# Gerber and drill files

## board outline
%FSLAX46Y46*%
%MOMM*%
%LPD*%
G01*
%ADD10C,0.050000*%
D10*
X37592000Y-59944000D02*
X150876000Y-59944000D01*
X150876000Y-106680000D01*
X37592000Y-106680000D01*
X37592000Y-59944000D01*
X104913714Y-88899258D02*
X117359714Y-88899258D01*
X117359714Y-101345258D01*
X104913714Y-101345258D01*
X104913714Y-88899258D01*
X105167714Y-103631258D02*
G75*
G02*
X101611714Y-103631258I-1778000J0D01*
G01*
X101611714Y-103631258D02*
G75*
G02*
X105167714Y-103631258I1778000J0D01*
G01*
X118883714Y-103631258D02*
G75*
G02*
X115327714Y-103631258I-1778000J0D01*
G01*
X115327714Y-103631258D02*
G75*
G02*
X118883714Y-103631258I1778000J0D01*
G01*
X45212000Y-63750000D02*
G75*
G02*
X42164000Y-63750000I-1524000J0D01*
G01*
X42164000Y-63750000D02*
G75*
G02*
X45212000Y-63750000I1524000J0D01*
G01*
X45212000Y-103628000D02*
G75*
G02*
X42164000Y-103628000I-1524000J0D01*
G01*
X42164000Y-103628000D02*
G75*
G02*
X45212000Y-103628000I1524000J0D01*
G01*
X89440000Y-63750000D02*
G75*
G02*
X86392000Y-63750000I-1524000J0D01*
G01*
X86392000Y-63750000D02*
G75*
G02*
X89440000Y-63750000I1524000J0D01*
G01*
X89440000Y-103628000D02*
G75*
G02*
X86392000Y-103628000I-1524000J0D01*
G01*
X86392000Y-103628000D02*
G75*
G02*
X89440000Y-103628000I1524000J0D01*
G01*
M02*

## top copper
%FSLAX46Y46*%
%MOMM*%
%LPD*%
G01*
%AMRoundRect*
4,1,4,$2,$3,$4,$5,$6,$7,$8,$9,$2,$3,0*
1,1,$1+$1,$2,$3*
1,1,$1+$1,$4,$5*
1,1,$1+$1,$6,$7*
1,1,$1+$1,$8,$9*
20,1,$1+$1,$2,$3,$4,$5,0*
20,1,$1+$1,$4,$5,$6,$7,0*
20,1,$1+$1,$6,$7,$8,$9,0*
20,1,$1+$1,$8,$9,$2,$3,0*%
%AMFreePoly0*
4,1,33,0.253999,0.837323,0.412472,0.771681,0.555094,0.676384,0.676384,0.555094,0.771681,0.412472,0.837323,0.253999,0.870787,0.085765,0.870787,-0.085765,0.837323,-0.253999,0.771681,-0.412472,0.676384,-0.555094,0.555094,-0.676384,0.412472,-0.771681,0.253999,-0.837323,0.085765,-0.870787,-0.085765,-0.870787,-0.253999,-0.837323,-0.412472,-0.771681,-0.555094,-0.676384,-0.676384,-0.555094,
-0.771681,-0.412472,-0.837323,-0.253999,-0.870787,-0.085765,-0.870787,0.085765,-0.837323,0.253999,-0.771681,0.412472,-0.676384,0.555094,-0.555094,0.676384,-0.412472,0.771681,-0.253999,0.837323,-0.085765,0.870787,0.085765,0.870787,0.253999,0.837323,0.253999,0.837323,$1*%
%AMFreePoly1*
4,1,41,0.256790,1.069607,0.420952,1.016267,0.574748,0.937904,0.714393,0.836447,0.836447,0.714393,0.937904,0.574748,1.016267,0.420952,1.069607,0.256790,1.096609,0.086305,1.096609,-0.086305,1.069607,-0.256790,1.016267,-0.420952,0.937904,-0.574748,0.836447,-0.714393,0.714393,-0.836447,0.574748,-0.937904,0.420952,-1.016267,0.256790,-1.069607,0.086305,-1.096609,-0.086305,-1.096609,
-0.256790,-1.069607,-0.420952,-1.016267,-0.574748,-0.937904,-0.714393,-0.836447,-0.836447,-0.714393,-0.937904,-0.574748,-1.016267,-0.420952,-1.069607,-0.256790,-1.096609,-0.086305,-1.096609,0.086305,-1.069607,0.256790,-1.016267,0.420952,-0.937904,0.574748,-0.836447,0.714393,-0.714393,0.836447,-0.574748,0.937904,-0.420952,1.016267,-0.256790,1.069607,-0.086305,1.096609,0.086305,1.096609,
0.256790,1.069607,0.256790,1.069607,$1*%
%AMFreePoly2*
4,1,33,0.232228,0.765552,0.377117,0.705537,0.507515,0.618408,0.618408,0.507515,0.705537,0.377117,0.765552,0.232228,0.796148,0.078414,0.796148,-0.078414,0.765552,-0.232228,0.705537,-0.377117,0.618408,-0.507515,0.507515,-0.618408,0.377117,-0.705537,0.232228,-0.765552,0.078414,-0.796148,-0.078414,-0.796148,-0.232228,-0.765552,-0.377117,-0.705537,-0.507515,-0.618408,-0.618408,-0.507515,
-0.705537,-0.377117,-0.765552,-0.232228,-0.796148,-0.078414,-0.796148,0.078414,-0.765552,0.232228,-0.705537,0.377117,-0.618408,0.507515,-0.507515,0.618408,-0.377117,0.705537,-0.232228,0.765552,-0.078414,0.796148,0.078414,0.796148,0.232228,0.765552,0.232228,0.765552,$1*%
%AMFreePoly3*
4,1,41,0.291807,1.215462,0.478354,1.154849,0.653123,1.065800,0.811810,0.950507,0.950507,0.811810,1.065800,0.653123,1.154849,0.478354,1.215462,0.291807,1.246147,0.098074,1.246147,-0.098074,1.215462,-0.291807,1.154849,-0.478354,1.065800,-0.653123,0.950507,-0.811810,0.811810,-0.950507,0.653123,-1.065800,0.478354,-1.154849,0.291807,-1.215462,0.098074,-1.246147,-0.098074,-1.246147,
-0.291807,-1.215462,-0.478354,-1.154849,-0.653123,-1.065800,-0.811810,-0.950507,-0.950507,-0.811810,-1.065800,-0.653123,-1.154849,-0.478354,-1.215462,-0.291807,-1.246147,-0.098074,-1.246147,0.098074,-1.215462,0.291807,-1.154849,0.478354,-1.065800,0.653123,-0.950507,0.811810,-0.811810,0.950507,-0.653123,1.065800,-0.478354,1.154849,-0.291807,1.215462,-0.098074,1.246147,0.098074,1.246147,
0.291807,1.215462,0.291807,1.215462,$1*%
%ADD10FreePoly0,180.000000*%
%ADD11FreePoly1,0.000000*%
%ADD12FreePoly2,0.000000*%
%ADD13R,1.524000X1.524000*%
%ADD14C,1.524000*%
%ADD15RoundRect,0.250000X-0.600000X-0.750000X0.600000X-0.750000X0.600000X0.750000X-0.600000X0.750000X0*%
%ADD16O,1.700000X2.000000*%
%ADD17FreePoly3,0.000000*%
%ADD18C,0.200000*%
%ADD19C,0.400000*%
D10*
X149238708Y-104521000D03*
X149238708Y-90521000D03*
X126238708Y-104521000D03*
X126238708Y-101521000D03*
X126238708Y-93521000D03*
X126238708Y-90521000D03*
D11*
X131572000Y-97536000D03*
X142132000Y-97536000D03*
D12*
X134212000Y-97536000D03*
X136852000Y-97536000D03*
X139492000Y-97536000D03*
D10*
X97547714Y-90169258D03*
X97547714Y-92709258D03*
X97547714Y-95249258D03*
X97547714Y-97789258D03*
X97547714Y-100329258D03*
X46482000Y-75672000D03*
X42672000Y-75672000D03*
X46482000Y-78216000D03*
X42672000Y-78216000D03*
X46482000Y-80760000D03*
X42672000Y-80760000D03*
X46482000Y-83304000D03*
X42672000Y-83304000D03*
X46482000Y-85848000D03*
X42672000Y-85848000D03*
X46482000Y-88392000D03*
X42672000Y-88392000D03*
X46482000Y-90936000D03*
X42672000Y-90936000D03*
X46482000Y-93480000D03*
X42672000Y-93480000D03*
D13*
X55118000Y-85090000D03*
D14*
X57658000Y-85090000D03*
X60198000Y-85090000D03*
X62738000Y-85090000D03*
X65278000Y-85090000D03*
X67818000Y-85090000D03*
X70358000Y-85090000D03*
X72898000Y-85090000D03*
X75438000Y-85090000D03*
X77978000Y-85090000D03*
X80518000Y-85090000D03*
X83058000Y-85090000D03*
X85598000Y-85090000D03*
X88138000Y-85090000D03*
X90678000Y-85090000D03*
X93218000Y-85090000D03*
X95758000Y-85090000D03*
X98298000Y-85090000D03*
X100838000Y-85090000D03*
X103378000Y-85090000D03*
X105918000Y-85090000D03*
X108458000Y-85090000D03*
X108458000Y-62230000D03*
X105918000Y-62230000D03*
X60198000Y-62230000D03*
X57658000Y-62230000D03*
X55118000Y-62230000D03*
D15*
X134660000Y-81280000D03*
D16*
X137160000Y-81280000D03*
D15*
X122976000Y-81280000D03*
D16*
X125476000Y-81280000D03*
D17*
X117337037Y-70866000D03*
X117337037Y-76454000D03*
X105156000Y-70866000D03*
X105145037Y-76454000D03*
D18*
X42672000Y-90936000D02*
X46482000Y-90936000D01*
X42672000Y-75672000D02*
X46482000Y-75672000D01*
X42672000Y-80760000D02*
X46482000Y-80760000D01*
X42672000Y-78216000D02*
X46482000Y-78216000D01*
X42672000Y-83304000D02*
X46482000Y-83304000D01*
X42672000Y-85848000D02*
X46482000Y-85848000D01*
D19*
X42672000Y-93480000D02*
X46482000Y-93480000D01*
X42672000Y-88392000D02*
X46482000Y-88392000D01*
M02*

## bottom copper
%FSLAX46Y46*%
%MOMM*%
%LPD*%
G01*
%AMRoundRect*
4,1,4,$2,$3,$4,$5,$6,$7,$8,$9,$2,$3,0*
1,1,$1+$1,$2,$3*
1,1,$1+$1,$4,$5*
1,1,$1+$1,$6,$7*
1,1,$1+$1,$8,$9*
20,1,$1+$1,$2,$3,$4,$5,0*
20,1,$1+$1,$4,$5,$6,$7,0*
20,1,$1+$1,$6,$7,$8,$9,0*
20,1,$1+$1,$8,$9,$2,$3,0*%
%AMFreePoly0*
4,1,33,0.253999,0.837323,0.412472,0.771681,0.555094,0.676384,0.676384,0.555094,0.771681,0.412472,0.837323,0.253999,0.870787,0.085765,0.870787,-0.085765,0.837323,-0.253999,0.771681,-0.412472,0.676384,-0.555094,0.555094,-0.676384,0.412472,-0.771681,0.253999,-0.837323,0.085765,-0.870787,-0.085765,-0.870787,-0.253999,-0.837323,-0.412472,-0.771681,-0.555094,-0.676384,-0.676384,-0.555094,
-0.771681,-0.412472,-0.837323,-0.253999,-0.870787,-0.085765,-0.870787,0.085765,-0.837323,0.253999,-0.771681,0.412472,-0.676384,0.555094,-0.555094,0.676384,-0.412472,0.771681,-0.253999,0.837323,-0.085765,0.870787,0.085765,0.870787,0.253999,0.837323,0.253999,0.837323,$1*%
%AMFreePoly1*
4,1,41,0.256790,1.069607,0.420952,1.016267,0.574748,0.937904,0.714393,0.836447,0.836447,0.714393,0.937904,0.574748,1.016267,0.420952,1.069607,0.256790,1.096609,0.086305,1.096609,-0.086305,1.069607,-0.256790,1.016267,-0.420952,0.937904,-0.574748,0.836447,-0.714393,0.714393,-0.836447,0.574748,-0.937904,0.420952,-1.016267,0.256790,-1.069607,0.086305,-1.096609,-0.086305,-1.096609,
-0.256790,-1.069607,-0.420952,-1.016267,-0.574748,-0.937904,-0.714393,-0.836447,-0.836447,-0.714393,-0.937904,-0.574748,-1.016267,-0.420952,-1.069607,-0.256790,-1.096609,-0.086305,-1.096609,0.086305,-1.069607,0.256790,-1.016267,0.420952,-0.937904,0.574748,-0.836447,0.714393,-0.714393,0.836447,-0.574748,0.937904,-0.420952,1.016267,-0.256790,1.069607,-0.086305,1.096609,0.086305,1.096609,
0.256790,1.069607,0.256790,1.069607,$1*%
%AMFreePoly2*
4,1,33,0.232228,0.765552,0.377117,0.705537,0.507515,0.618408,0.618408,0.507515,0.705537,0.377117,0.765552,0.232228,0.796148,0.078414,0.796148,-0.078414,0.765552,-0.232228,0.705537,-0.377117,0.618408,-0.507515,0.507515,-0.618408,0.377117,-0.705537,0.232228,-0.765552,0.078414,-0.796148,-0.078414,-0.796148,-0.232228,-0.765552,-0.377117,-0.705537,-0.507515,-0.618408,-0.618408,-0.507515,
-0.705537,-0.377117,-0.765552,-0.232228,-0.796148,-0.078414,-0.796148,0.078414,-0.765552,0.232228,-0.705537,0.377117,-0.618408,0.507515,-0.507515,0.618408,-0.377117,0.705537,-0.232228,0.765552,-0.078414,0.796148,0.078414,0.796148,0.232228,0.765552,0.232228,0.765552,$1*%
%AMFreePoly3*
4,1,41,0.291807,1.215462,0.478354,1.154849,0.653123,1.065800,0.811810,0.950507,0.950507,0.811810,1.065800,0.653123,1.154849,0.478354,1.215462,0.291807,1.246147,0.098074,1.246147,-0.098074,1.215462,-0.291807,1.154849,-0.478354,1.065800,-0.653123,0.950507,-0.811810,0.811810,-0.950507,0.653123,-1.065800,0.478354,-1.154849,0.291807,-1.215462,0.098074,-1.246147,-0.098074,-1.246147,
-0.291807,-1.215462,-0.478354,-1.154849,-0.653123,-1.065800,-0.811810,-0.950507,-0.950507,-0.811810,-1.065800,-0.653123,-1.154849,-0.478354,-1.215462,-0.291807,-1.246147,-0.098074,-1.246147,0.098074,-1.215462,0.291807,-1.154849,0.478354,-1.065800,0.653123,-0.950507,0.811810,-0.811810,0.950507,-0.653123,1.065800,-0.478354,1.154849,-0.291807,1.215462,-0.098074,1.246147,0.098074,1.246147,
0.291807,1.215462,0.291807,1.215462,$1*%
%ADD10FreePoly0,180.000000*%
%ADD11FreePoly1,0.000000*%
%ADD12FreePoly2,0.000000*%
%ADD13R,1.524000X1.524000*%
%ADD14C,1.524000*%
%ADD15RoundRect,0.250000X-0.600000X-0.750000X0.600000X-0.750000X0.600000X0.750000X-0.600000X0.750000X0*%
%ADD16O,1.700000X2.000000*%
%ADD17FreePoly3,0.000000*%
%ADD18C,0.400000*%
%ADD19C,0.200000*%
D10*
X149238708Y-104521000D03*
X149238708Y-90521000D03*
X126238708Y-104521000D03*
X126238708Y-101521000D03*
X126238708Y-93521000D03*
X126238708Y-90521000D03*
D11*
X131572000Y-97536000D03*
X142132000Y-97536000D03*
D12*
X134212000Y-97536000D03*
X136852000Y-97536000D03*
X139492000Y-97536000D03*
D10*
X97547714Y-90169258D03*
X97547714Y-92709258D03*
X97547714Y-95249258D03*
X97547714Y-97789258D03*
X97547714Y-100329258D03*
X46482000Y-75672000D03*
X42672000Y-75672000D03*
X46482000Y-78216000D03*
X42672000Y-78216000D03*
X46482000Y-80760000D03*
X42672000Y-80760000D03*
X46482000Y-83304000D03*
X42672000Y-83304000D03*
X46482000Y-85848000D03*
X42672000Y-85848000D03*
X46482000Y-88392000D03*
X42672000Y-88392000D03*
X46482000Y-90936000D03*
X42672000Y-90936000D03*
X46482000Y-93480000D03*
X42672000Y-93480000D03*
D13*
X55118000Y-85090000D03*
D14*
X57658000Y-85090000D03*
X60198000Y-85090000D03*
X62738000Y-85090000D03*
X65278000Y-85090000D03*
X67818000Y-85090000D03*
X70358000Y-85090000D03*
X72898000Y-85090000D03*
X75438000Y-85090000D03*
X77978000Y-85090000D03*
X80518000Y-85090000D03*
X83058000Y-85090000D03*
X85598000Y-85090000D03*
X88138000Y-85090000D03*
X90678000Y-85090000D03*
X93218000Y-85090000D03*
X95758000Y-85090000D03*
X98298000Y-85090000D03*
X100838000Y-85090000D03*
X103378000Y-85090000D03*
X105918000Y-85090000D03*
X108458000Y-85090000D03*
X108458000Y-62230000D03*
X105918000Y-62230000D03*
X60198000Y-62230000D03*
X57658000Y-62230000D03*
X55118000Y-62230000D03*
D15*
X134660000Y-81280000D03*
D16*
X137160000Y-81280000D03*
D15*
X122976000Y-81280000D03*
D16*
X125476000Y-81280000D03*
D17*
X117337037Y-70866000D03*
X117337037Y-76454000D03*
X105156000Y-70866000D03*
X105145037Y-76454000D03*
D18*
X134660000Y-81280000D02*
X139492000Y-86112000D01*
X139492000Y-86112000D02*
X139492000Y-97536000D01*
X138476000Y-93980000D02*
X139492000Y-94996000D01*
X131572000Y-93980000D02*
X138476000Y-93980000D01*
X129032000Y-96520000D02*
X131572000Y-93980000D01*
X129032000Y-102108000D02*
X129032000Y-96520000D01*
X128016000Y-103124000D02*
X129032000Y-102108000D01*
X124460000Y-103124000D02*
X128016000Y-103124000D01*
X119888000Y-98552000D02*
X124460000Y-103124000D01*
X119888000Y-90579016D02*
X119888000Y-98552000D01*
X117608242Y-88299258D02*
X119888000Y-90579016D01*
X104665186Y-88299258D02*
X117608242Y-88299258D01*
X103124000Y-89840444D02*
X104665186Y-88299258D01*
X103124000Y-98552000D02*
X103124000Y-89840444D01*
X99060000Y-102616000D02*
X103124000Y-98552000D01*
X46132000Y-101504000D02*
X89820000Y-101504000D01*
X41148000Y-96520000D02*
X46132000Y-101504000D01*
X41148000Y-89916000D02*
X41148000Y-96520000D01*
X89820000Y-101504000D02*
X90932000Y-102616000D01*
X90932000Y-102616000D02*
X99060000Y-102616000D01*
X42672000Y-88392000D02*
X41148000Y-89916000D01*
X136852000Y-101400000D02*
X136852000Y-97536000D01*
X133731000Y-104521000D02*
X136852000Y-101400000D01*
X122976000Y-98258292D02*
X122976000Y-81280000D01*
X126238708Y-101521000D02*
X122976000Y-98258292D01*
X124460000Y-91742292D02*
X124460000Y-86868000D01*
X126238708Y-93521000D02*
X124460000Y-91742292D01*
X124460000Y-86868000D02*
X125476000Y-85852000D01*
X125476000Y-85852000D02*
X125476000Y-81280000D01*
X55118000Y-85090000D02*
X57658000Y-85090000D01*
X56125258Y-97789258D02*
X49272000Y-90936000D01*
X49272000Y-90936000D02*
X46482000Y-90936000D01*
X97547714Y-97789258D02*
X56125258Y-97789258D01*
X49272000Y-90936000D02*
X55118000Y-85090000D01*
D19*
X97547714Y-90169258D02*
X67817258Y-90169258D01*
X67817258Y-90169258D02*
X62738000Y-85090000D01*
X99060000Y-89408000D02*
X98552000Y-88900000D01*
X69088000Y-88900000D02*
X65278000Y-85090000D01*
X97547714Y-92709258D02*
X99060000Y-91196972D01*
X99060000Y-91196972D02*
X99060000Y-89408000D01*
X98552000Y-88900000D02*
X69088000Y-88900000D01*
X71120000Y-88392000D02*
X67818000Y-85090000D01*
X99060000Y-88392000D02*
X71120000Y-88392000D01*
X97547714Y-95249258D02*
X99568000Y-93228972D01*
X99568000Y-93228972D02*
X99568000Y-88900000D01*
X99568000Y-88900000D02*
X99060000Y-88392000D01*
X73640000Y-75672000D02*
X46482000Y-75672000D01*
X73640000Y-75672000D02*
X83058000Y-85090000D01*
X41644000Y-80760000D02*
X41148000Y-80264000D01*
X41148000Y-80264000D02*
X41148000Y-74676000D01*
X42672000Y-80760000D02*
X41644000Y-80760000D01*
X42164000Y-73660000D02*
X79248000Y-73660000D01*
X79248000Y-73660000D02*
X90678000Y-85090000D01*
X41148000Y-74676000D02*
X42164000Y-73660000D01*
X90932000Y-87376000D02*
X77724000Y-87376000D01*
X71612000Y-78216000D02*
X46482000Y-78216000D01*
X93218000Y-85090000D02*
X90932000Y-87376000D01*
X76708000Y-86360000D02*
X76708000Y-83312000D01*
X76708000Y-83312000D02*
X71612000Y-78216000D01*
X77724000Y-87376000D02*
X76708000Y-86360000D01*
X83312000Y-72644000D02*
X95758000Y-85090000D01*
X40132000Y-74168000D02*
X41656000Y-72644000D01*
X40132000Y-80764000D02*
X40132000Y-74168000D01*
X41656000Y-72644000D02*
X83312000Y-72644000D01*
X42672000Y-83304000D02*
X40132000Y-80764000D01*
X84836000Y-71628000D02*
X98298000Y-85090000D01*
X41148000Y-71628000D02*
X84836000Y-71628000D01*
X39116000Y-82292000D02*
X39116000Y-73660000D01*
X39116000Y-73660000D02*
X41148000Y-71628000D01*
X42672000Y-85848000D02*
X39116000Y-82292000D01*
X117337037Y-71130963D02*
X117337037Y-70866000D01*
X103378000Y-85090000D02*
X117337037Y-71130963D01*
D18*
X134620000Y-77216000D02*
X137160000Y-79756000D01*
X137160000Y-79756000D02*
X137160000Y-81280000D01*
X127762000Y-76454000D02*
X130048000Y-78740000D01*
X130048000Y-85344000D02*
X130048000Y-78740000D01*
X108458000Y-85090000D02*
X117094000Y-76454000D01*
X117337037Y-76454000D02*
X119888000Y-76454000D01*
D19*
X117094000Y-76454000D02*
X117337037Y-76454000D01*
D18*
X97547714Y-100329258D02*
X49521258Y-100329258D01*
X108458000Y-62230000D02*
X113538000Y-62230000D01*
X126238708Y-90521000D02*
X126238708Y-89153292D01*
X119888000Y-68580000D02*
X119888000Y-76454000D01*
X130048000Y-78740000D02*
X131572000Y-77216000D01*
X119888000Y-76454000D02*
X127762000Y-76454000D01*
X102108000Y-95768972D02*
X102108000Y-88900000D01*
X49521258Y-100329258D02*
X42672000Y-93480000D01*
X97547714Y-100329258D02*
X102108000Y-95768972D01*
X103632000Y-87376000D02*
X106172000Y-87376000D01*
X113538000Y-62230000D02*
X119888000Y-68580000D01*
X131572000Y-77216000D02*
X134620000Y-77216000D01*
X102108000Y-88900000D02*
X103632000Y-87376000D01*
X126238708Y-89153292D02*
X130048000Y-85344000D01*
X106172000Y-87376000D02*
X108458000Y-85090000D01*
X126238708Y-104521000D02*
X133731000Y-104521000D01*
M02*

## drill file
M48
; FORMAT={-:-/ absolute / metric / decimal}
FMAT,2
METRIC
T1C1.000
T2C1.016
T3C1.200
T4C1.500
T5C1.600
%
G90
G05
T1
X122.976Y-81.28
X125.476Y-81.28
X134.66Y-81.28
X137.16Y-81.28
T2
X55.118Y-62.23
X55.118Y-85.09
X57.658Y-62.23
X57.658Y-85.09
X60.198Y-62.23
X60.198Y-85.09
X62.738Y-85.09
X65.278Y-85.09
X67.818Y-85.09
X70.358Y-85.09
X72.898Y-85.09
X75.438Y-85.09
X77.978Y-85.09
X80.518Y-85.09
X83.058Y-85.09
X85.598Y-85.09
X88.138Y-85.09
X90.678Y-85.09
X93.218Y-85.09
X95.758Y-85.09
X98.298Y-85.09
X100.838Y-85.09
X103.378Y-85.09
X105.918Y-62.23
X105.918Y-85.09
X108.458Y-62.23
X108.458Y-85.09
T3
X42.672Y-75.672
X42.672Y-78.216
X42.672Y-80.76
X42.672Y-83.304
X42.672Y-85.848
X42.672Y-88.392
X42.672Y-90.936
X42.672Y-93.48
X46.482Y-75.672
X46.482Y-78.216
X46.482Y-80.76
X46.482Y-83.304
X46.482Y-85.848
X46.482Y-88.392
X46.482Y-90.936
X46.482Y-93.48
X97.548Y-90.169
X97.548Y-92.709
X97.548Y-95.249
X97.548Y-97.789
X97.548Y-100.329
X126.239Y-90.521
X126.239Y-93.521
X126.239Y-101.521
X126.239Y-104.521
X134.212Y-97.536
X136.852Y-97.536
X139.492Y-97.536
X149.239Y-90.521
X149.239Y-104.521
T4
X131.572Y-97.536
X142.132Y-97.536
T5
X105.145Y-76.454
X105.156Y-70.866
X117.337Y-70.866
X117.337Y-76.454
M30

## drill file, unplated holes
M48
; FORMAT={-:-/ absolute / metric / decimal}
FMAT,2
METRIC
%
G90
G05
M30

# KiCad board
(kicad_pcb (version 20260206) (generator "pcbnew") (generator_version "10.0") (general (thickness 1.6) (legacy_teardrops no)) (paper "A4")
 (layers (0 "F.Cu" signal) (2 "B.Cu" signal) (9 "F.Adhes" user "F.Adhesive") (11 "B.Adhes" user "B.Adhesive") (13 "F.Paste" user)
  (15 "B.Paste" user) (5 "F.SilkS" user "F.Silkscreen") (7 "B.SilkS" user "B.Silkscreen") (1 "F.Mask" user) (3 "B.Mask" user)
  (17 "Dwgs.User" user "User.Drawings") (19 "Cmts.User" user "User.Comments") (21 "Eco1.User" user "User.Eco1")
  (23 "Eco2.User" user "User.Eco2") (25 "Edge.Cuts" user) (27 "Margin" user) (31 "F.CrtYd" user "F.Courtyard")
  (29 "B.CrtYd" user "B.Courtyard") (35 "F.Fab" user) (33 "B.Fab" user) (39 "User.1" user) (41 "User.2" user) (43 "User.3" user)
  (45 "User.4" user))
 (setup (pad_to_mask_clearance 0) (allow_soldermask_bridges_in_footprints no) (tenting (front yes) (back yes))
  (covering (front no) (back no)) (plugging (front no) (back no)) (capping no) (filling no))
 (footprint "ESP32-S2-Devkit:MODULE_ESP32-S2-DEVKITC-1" (layer "F.Cu") (at 85.088 73.66 90)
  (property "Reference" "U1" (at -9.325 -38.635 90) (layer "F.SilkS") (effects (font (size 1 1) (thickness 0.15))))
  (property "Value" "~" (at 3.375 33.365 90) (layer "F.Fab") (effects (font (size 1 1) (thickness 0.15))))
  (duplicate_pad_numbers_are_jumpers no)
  (pad "1" thru_hole rect (at -11.43 -29.97 90) (size 1.524 1.524) (drill 1.016) (layers "*.Cu" "*.Mask") (remove_unused_layers no)
   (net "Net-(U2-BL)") (solder_mask_margin 0.102))
  (pad "2" thru_hole circle (at -11.43 -27.43 90) (size 1.524 1.524) (drill 1.016) (layers "*.Cu" "*.Mask") (remove_unused_layers no)
   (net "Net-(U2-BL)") (solder_mask_margin 0.102))
  (pad "3" thru_hole circle (at -11.43 -24.89 90) (size 1.524 1.524) (drill 1.016) (layers "*.Cu" "*.Mask") (remove_unused_layers no)
   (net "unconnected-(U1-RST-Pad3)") (solder_mask_margin 0.102))
  (pad "4" thru_hole circle (at -11.43 -22.35 90) (size 1.524 1.524) (drill 1.016) (layers "*.Cu" "*.Mask") (remove_unused_layers no)
   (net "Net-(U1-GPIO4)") (solder_mask_margin 0.102))
  (pad "5" thru_hole circle (at -11.43 -19.81 90) (size 1.524 1.524) (drill 1.016) (layers "*.Cu" "*.Mask") (remove_unused_layers no)
   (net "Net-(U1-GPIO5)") (solder_mask_margin 0.102))
  (pad "6" thru_hole circle (at -11.43 -17.27 90) (size 1.524 1.524) (drill 1.016) (layers "*.Cu" "*.Mask") (remove_unused_layers no)
   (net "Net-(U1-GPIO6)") (solder_mask_margin 0.102))
  (pad "7" thru_hole circle (at -11.43 -14.73 90) (size 1.524 1.524) (drill 1.016) (layers "*.Cu" "*.Mask") (remove_unused_layers no)
   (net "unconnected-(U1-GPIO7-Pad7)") (solder_mask_margin 0.102))
  (pad "8" thru_hole circle (at -11.43 -12.19 90) (size 1.524 1.524) (drill 1.016) (layers "*.Cu" "*.Mask") (remove_unused_layers no)
   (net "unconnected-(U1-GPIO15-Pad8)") (solder_mask_margin 0.102))
  (pad "9" thru_hole circle (at -11.43 -9.65 90) (size 1.524 1.524) (drill 1.016) (layers "*.Cu" "*.Mask") (remove_unused_layers no)
   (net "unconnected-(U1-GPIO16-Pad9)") (solder_mask_margin 0.102))
  (pad "10" thru_hole circle (at -11.43 -7.11 90) (size 1.524 1.524) (drill 1.016) (layers "*.Cu" "*.Mask") (remove_unused_layers no)
   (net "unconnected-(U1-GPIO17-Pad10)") (solder_mask_margin 0.102))
  (pad "11" thru_hole circle (at -11.43 -4.57 90) (size 1.524 1.524) (drill 1.016) (layers "*.Cu" "*.Mask") (remove_unused_layers no)
   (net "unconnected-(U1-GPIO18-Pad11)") (solder_mask_margin 0.102))
  (pad "12" thru_hole circle (at -11.43 -2.03 90) (size 1.524 1.524) (drill 1.016) (layers "*.Cu" "*.Mask") (remove_unused_layers no)
   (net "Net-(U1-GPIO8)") (solder_mask_margin 0.102))
  (pad "13" thru_hole circle (at -11.43 0.51 90) (size 1.524 1.524) (drill 1.016) (layers "*.Cu" "*.Mask") (remove_unused_layers no)
   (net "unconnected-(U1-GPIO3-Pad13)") (solder_mask_margin 0.102))
  (pad "14" thru_hole circle (at -11.43 3.05 90) (size 1.524 1.524) (drill 1.016) (layers "*.Cu" "*.Mask") (remove_unused_layers no)
   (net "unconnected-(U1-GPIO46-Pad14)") (solder_mask_margin 0.102))
  (pad "15" thru_hole circle (at -11.43 5.59 90) (size 1.524 1.524) (drill 1.016) (layers "*.Cu" "*.Mask") (remove_unused_layers no)
   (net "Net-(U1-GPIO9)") (solder_mask_margin 0.102))
  (pad "16" thru_hole circle (at -11.43 8.13 90) (size 1.524 1.524) (drill 1.016) (layers "*.Cu" "*.Mask") (remove_unused_layers no)
   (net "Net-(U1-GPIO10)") (solder_mask_margin 0.102))
  (pad "17" thru_hole circle (at -11.43 10.67 90) (size 1.524 1.524) (drill 1.016) (layers "*.Cu" "*.Mask") (remove_unused_layers no)
   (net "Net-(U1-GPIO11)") (solder_mask_margin 0.102))
  (pad "18" thru_hole circle (at -11.43 13.21 90) (size 1.524 1.524) (drill 1.016) (layers "*.Cu" "*.Mask") (remove_unused_layers no)
   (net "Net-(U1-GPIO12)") (solder_mask_margin 0.102))
  (pad "19" thru_hole circle (at -11.43 15.75 90) (size 1.524 1.524) (drill 1.016) (layers "*.Cu" "*.Mask") (remove_unused_layers no)
   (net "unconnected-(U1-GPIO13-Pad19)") (solder_mask_margin 0.102))
  (pad "20" thru_hole circle (at -11.43 18.29 90) (size 1.524 1.524) (drill 1.016) (layers "*.Cu" "*.Mask") (remove_unused_layers no)
   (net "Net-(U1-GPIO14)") (solder_mask_margin 0.102))
  (pad "21" thru_hole circle (at -11.43 20.83 90) (size 1.524 1.524) (drill 1.016) (layers "*.Cu" "*.Mask") (remove_unused_layers no)
   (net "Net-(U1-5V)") (solder_mask_margin 0.102))
  (pad "22" thru_hole circle (at -11.43 23.37 90) (size 1.524 1.524) (drill 1.016) (layers "*.Cu" "*.Mask") (remove_unused_layers no)
   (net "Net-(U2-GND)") (solder_mask_margin 0.102))
  (pad "23" thru_hole circle (at 11.43 23.37 90) (size 1.524 1.524) (drill 1.016) (layers "*.Cu" "*.Mask") (remove_unused_layers no)
   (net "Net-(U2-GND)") (solder_mask_margin 0.102))
  (pad "24" thru_hole circle (at 11.43 20.83 90) (size 1.524 1.524) (drill 1.016) (layers "*.Cu" "*.Mask") (remove_unused_layers no)
   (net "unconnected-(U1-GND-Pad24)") (solder_mask_margin 0.102))
  (pad "42" thru_hole circle (at 11.43 -24.89 90) (size 1.524 1.524) (drill 1.016) (layers "*.Cu" "*.Mask") (remove_unused_layers no)
   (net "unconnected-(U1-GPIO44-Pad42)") (solder_mask_margin 0.102))
  (pad "43" thru_hole circle (at 11.43 -27.43 90) (size 1.524 1.524) (drill 1.016) (layers "*.Cu" "*.Mask") (remove_unused_layers no)
   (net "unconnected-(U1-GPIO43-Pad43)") (solder_mask_margin 0.102))
  (pad "44" thru_hole circle (at 11.43 -29.97 90) (size 1.524 1.524) (drill 1.016) (layers "*.Cu" "*.Mask") (remove_unused_layers no)
   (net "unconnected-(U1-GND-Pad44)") (solder_mask_margin 0.102)))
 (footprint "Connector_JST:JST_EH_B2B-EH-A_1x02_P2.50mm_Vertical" (layer "F.Cu") (at 134.66 81.28)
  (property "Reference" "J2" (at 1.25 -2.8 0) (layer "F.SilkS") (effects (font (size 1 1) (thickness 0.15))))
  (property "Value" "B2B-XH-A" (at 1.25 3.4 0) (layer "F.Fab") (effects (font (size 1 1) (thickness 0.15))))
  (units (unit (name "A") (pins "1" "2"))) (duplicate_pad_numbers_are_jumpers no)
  (pad "1" thru_hole roundrect (at 0 0) (size 1.7 2) (drill 1) (layers "*.Cu" "*.Mask") (remove_unused_layers no)
   (roundrect_rratio 0.147059) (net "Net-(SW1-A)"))
  (pad "2" thru_hole oval (at 2.5 0) (size 1.7 2) (drill 1) (layers "*.Cu" "*.Mask") (remove_unused_layers no) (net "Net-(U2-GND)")))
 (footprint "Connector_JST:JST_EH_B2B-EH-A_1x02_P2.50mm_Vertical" (layer "F.Cu") (at 122.976 81.28)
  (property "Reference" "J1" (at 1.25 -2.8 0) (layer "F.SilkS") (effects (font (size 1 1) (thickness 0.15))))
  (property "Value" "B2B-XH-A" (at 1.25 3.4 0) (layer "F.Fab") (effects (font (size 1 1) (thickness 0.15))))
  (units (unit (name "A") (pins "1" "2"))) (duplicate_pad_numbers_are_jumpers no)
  (pad "1" thru_hole roundrect (at 0 0) (size 1.7 2) (drill 1) (layers "*.Cu" "*.Mask") (remove_unused_layers no)
   (roundrect_rratio 0.147059) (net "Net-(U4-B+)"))
  (pad "2" thru_hole oval (at 2.5 0) (size 1.7 2) (drill 1) (layers "*.Cu" "*.Mask") (remove_unused_layers no) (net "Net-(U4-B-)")))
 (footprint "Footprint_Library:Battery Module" (layer "F.Cu") (at 126.238708 104.521 180)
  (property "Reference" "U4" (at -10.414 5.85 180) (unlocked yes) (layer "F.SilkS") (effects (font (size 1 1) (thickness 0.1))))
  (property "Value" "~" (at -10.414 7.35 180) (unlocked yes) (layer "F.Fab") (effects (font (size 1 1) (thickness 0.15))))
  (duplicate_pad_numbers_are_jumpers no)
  (pad "1" thru_hole custom (at -23 0 180) (size 1.75 1.75) (drill 1.2) (layers "*.Cu" "*.Mask") (remove_unused_layers no)
   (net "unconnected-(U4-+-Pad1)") (thermal_bridge_angle 90) (options (clearance outline) (anchor circle)) (primitives))
  (pad "2" thru_hole custom (at -23 14 180) (size 1.75 1.75) (drill 1.2) (layers "*.Cu" "*.Mask") (remove_unused_layers no)
   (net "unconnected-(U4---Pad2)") (thermal_bridge_angle 90) (options (clearance outline) (anchor circle)) (primitives))
  (pad "3" thru_hole custom (at 0 0 180) (size 1.75 1.75) (drill 1.2) (layers "*.Cu" "*.Mask") (remove_unused_layers no) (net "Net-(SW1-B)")
   (thermal_bridge_angle 90) (options (clearance outline) (anchor circle)) (primitives))
  (pad "4" thru_hole custom (at 0 3 180) (size 1.75 1.75) (drill 1.2) (layers "*.Cu" "*.Mask") (remove_unused_layers no) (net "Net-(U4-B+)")
   (thermal_bridge_angle 90) (options (clearance outline) (anchor circle)) (primitives))
  (pad "5" thru_hole custom (at 0 11 180) (size 1.75 1.75) (drill 1.2) (layers "*.Cu" "*.Mask") (remove_unused_layers no)
   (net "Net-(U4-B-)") (thermal_bridge_angle 90) (options (clearance outline) (anchor circle)) (primitives))
  (pad "6" thru_hole custom (at 0 14 180) (size 1.75 1.75) (drill 1.2) (layers "*.Cu" "*.Mask") (remove_unused_layers no)
   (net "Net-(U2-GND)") (thermal_bridge_angle 90) (options (clearance outline) (anchor circle)) (primitives)))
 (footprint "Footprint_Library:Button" (layer "F.Cu") (at 111.252 73.66)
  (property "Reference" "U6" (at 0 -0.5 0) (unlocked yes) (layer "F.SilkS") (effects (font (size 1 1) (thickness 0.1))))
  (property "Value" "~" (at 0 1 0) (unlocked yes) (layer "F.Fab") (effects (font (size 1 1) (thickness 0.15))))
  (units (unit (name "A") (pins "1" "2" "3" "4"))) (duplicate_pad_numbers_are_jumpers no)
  (pad "1" thru_hole custom (at 6.085037 -2.794) (size 2.5 2.5) (drill 1.6) (layers "*.Cu" "*.Mask") (remove_unused_layers no)
   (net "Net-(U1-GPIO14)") (thermal_bridge_angle 90) (options (clearance outline) (anchor circle)) (primitives))
  (pad "2" thru_hole custom (at 6.085037 2.794) (size 2.5 2.5) (drill 1.6) (layers "*.Cu" "*.Mask") (remove_unused_layers no)
   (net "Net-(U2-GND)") (thermal_bridge_angle 90) (options (clearance outline) (anchor circle)) (primitives))
  (pad "3" thru_hole custom (at -6.096 -2.794) (size 2.5 2.5) (drill 1.6) (layers "*.Cu" "*.Mask") (remove_unused_layers no)
   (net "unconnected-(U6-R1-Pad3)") (thermal_bridge_angle 90) (options (clearance outline) (anchor circle)) (primitives))
  (pad "4" thru_hole custom (at -6.106963 2.794) (size 2.5 2.5) (drill 1.6) (layers "*.Cu" "*.Mask") (remove_unused_layers no)
   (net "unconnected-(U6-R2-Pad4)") (thermal_bridge_angle 90) (options (clearance outline) (anchor circle)) (primitives)))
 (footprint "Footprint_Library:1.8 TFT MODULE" (layer "B.Cu") (at 42.672 74.672 180)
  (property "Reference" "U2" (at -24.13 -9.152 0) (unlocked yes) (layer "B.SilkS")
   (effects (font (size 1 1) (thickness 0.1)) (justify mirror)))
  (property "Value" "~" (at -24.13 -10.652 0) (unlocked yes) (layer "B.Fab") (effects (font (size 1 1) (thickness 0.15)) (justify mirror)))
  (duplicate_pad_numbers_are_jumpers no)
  (fp_circle (center -1.016 10.922) (end 0.508 10.922) (stroke (width 0.05) (type default)) (fill no) (layer "Edge.Cuts"))
  (fp_circle (center -1.016 -28.956) (end 0.508 -28.956) (stroke (width 0.05) (type default)) (fill no) (layer "Edge.Cuts"))
  (fp_circle (center -45.244 10.922) (end -43.72 10.922) (stroke (width 0.05) (type solid)) (fill no) (layer "Edge.Cuts"))
  (fp_circle (center -45.244 -28.956) (end -43.72 -28.956) (stroke (width 0.05) (type solid)) (fill no) (layer "Edge.Cuts"))
  (pad "1" thru_hole custom (at -3.81 -1 180) (size 1.75 1.75) (drill 1.2) (layers "*.Cu" "*.Mask") (remove_unused_layers no)
   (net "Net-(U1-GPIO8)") (thermal_bridge_angle 90) (options (clearance outline) (anchor circle)) (primitives))
  (pad "1" thru_hole custom (at 0 -1 180) (size 1.75 1.75) (drill 1.2) (layers "*.Cu" "*.Mask") (remove_unused_layers no)
   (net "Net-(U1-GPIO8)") (thermal_bridge_angle 90) (options (clearance outline) (anchor circle)) (primitives))
  (pad "2" thru_hole custom (at -3.81 -3.544 180) (size 1.75 1.75) (drill 1.2) (layers "*.Cu" "*.Mask") (remove_unused_layers no)
   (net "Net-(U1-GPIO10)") (thermal_bridge_angle 90) (options (clearance outline) (anchor circle)) (primitives))
  (pad "2" thru_hole custom (at 0 -3.544 180) (size 1.75 1.75) (drill 1.2) (layers "*.Cu" "*.Mask") (remove_unused_layers no)
   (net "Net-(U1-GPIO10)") (thermal_bridge_angle 90) (options (clearance outline) (anchor circle)) (primitives))
  (pad "3" thru_hole custom (at -3.81 -6.088 180) (size 1.75 1.75) (drill 1.2) (layers "*.Cu" "*.Mask") (remove_unused_layers no)
   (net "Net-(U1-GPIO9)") (thermal_bridge_angle 90) (options (clearance outline) (anchor circle)) (primitives))
  (pad "3" thru_hole custom (at 0 -6.088 180) (size 1.75 1.75) (drill 1.2) (layers "*.Cu" "*.Mask") (remove_unused_layers no)
   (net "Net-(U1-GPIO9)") (thermal_bridge_angle 90) (options (clearance outline) (anchor circle)) (primitives))
  (pad "4" thru_hole custom (at -3.81 -8.632 180) (size 1.75 1.75) (drill 1.2) (layers "*.Cu" "*.Mask") (remove_unused_layers no)
   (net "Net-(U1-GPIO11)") (thermal_bridge_angle 90) (options (clearance outline) (anchor circle)) (primitives))
  (pad "4" thru_hole custom (at 0 -8.632 180) (size 1.75 1.75) (drill 1.2) (layers "*.Cu" "*.Mask") (remove_unused_layers no)
   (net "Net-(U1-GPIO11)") (thermal_bridge_angle 90) (options (clearance outline) (anchor circle)) (primitives))
  (pad "5" thru_hole custom (at -3.81 -11.176 180) (size 1.75 1.75) (drill 1.2) (layers "*.Cu" "*.Mask") (remove_unused_layers no)
   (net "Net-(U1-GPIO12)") (thermal_bridge_angle 90) (options (clearance outline) (anchor circle)) (primitives))
  (pad "5" thru_hole custom (at 0 -11.176 180) (size 1.75 1.75) (drill 1.2) (layers "*.Cu" "*.Mask") (remove_unused_layers no)
   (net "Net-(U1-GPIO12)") (thermal_bridge_angle 90) (options (clearance outline) (anchor circle)) (primitives))
  (pad "6" thru_hole custom (at -3.81 -13.72 180) (size 1.75 1.75) (drill 1.2) (layers "*.Cu" "*.Mask") (remove_unused_layers no)
   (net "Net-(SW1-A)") (thermal_bridge_angle 90) (options (clearance outline) (anchor circle)) (primitives))
  (pad "6" thru_hole custom (at 0 -13.72 180) (size 1.75 1.75) (drill 1.2) (layers "*.Cu" "*.Mask") (remove_unused_layers no)
   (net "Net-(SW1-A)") (thermal_bridge_angle 90) (options (clearance outline) (anchor circle)) (primitives))
  (pad "7" thru_hole custom (at -3.81 -16.264 180) (size 1.75 1.75) (drill 1.2) (layers "*.Cu" "*.Mask") (remove_unused_layers no)
   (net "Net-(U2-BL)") (thermal_bridge_angle 90) (options (clearance outline) (anchor circle)) (primitives))
  (pad "7" thru_hole custom (at 0 -16.264 180) (size 1.75 1.75) (drill 1.2) (layers "*.Cu" "*.Mask") (remove_unused_layers no)
   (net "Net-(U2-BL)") (thermal_bridge_angle 90) (options (clearance outline) (anchor circle)) (primitives))
  (pad "8" thru_hole custom (at -3.81 -18.808 180) (size 1.75 1.75) (drill 1.2) (layers "*.Cu" "*.Mask") (remove_unused_layers no)
   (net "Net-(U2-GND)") (thermal_bridge_angle 90) (options (clearance outline) (anchor circle)) (primitives))
  (pad "8" thru_hole custom (at 0 -18.808 180) (size 1.75 1.75) (drill 1.2) (layers "*.Cu" "*.Mask") (remove_unused_layers no)
   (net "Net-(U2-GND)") (thermal_bridge_angle 90) (options (clearance outline) (anchor circle)) (primitives)))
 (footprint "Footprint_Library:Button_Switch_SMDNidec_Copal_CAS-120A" (layer "B.Cu") (at 131.572 97.536)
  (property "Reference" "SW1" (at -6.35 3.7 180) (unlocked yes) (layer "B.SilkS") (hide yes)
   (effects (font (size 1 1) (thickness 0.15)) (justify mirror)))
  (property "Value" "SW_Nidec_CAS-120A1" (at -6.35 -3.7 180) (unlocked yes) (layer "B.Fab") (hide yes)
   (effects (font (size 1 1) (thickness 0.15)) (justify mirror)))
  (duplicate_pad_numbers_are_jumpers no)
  (pad "0" thru_hole custom (at 0 0) (size 2.2 2.2) (drill 1.5) (layers "*.Cu" "*.Mask") (remove_unused_layers no) (thermal_bridge_angle 90)
   (options (clearance outline) (anchor circle)) (primitives))
  (pad "0" thru_hole custom (at 10.56 0) (size 2.2 2.2) (drill 1.5) (layers "*.Cu" "*.Mask") (remove_unused_layers no)
   (thermal_bridge_angle 90) (options (clearance outline) (anchor circle)) (primitives))
  (pad "1" thru_hole custom (at 2.64 0) (size 1.6 1.6) (drill 1.2) (layers "*.Cu" "*.Mask") (remove_unused_layers no)
   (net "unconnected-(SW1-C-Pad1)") (thermal_bridge_angle 90) (options (clearance outline) (anchor circle)) (primitives))
  (pad "2" thru_hole custom (at 5.28 0) (size 1.6 1.6) (drill 1.2) (layers "*.Cu" "*.Mask") (remove_unused_layers no) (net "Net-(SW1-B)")
   (thermal_bridge_angle 90) (options (clearance outline) (anchor circle)) (primitives))
  (pad "3" thru_hole custom (at 7.92 0) (size 1.6 1.6) (drill 1.2) (layers "*.Cu" "*.Mask") (remove_unused_layers no) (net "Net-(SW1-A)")
   (thermal_bridge_angle 90) (options (clearance outline) (anchor circle)) (primitives)))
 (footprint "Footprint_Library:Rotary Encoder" (layer "B.Cu") (at 97.547714 90.169258 180)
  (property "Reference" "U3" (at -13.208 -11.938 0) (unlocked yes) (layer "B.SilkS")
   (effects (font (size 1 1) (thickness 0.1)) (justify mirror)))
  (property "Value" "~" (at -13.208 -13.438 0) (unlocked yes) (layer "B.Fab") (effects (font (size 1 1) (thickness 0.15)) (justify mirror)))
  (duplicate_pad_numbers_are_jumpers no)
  (fp_rect (start -19.812 1.27) (end -7.366 -11.176) (stroke (width 0.05) (type default)) (fill no) (layer "Edge.Cuts"))
  (fp_circle (center -5.842 -13.462) (end -4.064 -13.462) (stroke (width 0.05) (type default)) (fill no) (layer "Edge.Cuts"))
  (fp_circle (center -19.558 -13.462) (end -17.78 -13.462) (stroke (width 0.05) (type default)) (fill no) (layer "Edge.Cuts"))
  (pad "1" thru_hole custom (at 0 0 180) (size 1.75 1.75) (drill 1.2) (layers "*.Cu" "*.Mask") (remove_unused_layers no)
   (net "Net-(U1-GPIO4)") (thermal_bridge_angle 90) (options (clearance outline) (anchor circle)) (primitives))
  (pad "2" thru_hole custom (at 0 -2.54 180) (size 1.75 1.75) (drill 1.2) (layers "*.Cu" "*.Mask") (remove_unused_layers no)
   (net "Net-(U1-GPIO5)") (thermal_bridge_angle 90) (options (clearance outline) (anchor circle)) (primitives))
  (pad "3" thru_hole custom (at 0 -5.08 180) (size 1.75 1.75) (drill 1.2) (layers "*.Cu" "*.Mask") (remove_unused_layers no)
   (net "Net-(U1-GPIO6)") (thermal_bridge_angle 90) (options (clearance outline) (anchor circle)) (primitives))
  (pad "4" thru_hole custom (at 0 -7.62 180) (size 1.75 1.75) (drill 1.2) (layers "*.Cu" "*.Mask") (remove_unused_layers no)
   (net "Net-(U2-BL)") (thermal_bridge_angle 90) (options (clearance outline) (anchor circle)) (primitives))
  (pad "5" thru_hole custom (at 0 -10.16 180) (size 1.75 1.75) (drill 1.2) (layers "*.Cu" "*.Mask") (remove_unused_layers no)
   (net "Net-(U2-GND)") (thermal_bridge_angle 90) (options (clearance outline) (anchor circle)) (primitives)))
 (gr_rect (start 37.592 59.944) (end 150.876 106.68) (stroke (width 0.05) (type default)) (fill no) (layer "Edge.Cuts"))
 (segment (start 42.672 90.936) (end 46.482 90.936) (width 0.2) (layer "F.Cu") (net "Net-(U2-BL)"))
 (segment (start 55.118 85.09) (end 57.658 85.09) (width 0.4) (layer "B.Cu") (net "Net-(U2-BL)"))
 (segment (start 56.125258 97.789258) (end 49.272 90.936) (width 0.4) (layer "B.Cu") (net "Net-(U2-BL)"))
 (segment (start 49.272 90.936) (end 46.482 90.936) (width 0.4) (layer "B.Cu") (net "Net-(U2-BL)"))
 (segment (start 97.547714 97.789258) (end 56.125258 97.789258) (width 0.4) (layer "B.Cu") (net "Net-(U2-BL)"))
 (segment (start 49.272 90.936) (end 55.118 85.09) (width 0.4) (layer "B.Cu") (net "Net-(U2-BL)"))
 (segment (start 97.547714 90.169258) (end 67.817258 90.169258) (width 0.2) (layer "B.Cu") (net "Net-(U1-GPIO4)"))
 (segment (start 67.817258 90.169258) (end 62.738 85.09) (width 0.2) (layer "B.Cu") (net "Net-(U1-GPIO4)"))
 (segment (start 99.06 89.408) (end 98.552 88.9) (width 0.2) (layer "B.Cu") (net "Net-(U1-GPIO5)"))
 (segment (start 69.088 88.9) (end 65.278 85.09) (width 0.2) (layer "B.Cu") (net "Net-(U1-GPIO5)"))
 (segment (start 97.547714 92.709258) (end 99.06 91.196972) (width 0.2) (layer "B.Cu") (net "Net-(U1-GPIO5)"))
 (segment (start 99.06 91.196972) (end 99.06 89.408) (width 0.2) (layer "B.Cu") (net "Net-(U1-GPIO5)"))
 (segment (start 98.552 88.9) (end 69.088 88.9) (width 0.2) (layer "B.Cu") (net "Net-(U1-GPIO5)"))
 (segment (start 71.12 88.392) (end 67.818 85.09) (width 0.2) (layer "B.Cu") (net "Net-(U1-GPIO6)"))
 (segment (start 99.06 88.392) (end 71.12 88.392) (width 0.2) (layer "B.Cu") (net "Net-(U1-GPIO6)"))
 (segment (start 97.547714 95.249258) (end 99.568 93.228972) (width 0.2) (layer "B.Cu") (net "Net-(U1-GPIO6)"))
 (segment (start 99.568 93.228972) (end 99.568 88.9) (width 0.2) (layer "B.Cu") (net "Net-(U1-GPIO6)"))
 (segment (start 99.568 88.9) (end 99.06 88.392) (width 0.2) (layer "B.Cu") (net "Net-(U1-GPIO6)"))
 (segment (start 42.672 75.672) (end 46.482 75.672) (width 0.2) (layer "F.Cu") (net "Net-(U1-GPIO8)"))
 (segment (start 73.64 75.672) (end 46.482 75.672) (width 0.2) (layer "B.Cu") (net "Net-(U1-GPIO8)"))
 (segment (start 73.64 75.672) (end 83.058 85.09) (width 0.2) (layer "B.Cu") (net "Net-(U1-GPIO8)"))
 (segment (start 42.672 80.76) (end 46.482 80.76) (width 0.2) (layer "F.Cu") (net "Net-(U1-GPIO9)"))
 (segment (start 41.644 80.76) (end 41.148 80.264) (width 0.2) (layer "B.Cu") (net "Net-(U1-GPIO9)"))
 (segment (start 41.148 80.264) (end 41.148 74.676) (width 0.2) (layer "B.Cu") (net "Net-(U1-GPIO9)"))
 (segment (start 42.672 80.76) (end 41.644 80.76) (width 0.2) (layer "B.Cu") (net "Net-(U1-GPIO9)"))
 (segment (start 42.164 73.66) (end 79.248 73.66) (width 0.2) (layer "B.Cu") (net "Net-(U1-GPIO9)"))
 (segment (start 79.248 73.66) (end 90.678 85.09) (width 0.2) (layer "B.Cu") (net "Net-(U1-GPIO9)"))
 (segment (start 41.148 74.676) (end 42.164 73.66) (width 0.2) (layer "B.Cu") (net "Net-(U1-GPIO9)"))
 (segment (start 42.672 78.216) (end 46.482 78.216) (width 0.2) (layer "F.Cu") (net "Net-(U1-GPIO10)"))
 (segment (start 90.932 87.376) (end 77.724 87.376) (width 0.2) (layer "B.Cu") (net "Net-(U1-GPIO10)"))
 (segment (start 71.612 78.216) (end 46.482 78.216) (width 0.2) (layer "B.Cu") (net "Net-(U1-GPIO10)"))
 (segment (start 93.218 85.09) (end 90.932 87.376) (width 0.2) (layer "B.Cu") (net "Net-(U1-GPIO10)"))
 (segment (start 76.708 86.36) (end 76.708 83.312) (width 0.2) (layer "B.Cu") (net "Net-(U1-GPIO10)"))
 (segment (start 76.708 83.312) (end 71.612 78.216) (width 0.2) (layer "B.Cu") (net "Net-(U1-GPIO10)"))
 (segment (start 77.724 87.376) (end 76.708 86.36) (width 0.2) (layer "B.Cu") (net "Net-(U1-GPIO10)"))
 (segment (start 42.672 83.304) (end 46.482 83.304) (width 0.2) (layer "F.Cu") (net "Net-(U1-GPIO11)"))
 (segment (start 83.312 72.644) (end 95.758 85.09) (width 0.2) (layer "B.Cu") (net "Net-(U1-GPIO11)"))
 (segment (start 40.132 74.168) (end 41.656 72.644) (width 0.2) (layer "B.Cu") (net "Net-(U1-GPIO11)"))
 (segment (start 40.132 80.764) (end 40.132 74.168) (width 0.2) (layer "B.Cu") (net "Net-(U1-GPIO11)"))
 (segment (start 41.656 72.644) (end 83.312 72.644) (width 0.2) (layer "B.Cu") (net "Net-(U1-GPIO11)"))
 (segment (start 42.672 83.304) (end 40.132 80.764) (width 0.2) (layer "B.Cu") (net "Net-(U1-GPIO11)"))
 (segment (start 42.672 85.848) (end 46.482 85.848) (width 0.2) (layer "F.Cu") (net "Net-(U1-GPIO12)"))
 (segment (start 84.836 71.628) (end 98.298 85.09) (width 0.2) (layer "B.Cu") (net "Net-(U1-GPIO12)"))
 (segment (start 41.148 71.628) (end 84.836 71.628) (width 0.2) (layer "B.Cu") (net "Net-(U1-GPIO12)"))
 (segment (start 39.116 82.292) (end 39.116 73.66) (width 0.2) (layer "B.Cu") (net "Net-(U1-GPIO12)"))
 (segment (start 39.116 73.66) (end 41.148 71.628) (width 0.2) (layer "B.Cu") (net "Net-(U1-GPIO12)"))
 (segment (start 42.672 85.848) (end 39.116 82.292) (width 0.2) (layer "B.Cu") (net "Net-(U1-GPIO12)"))
 (segment (start 117.337037 71.130963) (end 117.337037 70.866) (width 0.2) (layer "B.Cu") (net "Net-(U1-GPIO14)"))
 (segment (start 103.378 85.09) (end 117.337037 71.130963) (width 0.2) (layer "B.Cu") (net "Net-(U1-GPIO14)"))
 (segment (start 42.672 93.48) (end 46.482 93.48) (width 0.4) (layer "F.Cu") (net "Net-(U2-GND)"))
 (segment (start 134.62 77.216) (end 137.16 79.756) (width 0.4) (layer "B.Cu") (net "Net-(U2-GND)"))
 (segment (start 137.16 79.756) (end 137.16 81.28) (width 0.4) (layer "B.Cu") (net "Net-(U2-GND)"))
 (segment (start 127.762 76.454) (end 130.048 78.74) (width 0.4) (layer "B.Cu") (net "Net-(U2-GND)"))
 (segment (start 130.048 85.344) (end 130.048 78.74) (width 0.4) (layer "B.Cu") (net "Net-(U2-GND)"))
 (segment (start 108.458 85.09) (end 117.094 76.454) (width 0.4) (layer "B.Cu") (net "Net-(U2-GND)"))
 (segment (start 117.337037 76.454) (end 119.888 76.454) (width 0.4) (layer "B.Cu") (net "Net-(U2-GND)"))
 (segment (start 117.094 76.454) (end 117.337037 76.454) (width 0.2) (layer "B.Cu") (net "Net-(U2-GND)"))
 (segment (start 97.547714 100.329258) (end 49.521258 100.329258) (width 0.4) (layer "B.Cu") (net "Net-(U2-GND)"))
 (segment (start 108.458 62.23) (end 113.538 62.23) (width 0.4) (layer "B.Cu") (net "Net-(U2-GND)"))
 (segment (start 126.238708 90.521) (end 126.238708 89.153292) (width 0.4) (layer "B.Cu") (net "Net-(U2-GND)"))
 (segment (start 119.888 68.58) (end 119.888 76.454) (width 0.4) (layer "B.Cu") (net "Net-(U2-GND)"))
 (segment (start 130.048 78.74) (end 131.572 77.216) (width 0.4) (layer "B.Cu") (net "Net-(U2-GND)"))
 (segment (start 119.888 76.454) (end 127.762 76.454) (width 0.4) (layer "B.Cu") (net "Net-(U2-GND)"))
 (segment (start 102.108 95.768972) (end 102.108 88.9) (width 0.4) (layer "B.Cu") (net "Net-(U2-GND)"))
 (segment (start 49.521258 100.329258) (end 42.672 93.48) (width 0.4) (layer "B.Cu") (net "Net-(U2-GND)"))
 (segment (start 97.547714 100.329258) (end 102.108 95.768972) (width 0.4) (layer "B.Cu") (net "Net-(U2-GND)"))
 (segment (start 103.632 87.376) (end 106.172 87.376) (width 0.4) (layer "B.Cu") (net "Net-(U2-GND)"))
 (segment (start 113.538 62.23) (end 119.888 68.58) (width 0.4) (layer "B.Cu") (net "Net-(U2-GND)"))
 (segment (start 131.572 77.216) (end 134.62 77.216) (width 0.4) (layer "B.Cu") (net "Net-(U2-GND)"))
 (segment (start 102.108 88.9) (end 103.632 87.376) (width 0.4) (layer "B.Cu") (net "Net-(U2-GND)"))
 (segment (start 126.238708 89.153292) (end 130.048 85.344) (width 0.4) (layer "B.Cu") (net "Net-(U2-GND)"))
 (segment (start 106.172 87.376) (end 108.458 85.09) (width 0.4) (layer "B.Cu") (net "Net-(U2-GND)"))
 (segment (start 42.672 88.392) (end 46.482 88.392) (width 0.4) (layer "F.Cu") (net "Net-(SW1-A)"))
 (segment (start 103.124 98.552) (end 103.124 89.840444) (width 0.4) (layer "B.Cu") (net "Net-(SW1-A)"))
 (segment (start 128.016 103.124) (end 129.032 102.108) (width 0.4) (layer "B.Cu") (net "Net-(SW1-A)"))
 (segment (start 124.46 103.124) (end 128.016 103.124) (width 0.4) (layer "B.Cu") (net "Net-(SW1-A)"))
 (segment (start 139.492 86.112) (end 139.492 97.536) (width 0.4) (layer "B.Cu") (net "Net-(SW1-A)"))
 (segment (start 134.66 81.28) (end 139.492 86.112) (width 0.4) (layer "B.Cu") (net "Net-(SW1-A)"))
 (segment (start 131.572 93.98) (end 138.476 93.98) (width 0.4) (layer "B.Cu") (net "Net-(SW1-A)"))
 (segment (start 129.032 96.52) (end 131.572 93.98) (width 0.4) (layer "B.Cu") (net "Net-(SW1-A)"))
 (segment (start 119.888 98.552) (end 124.46 103.124) (width 0.4) (layer "B.Cu") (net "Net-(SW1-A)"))
 (segment (start 104.665186 88.299258) (end 117.608242 88.299258) (width 0.4) (layer "B.Cu") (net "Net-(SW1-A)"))
 (segment (start 99.06 102.616) (end 103.124 98.552) (width 0.4) (layer "B.Cu") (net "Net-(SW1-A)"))
 (segment (start 119.888 90.579016) (end 119.888 98.552) (width 0.4) (layer "B.Cu") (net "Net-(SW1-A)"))
 (segment (start 129.032 102.108) (end 129.032 96.52) (width 0.4) (layer "B.Cu") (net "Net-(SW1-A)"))
 (segment (start 138.476 93.98) (end 139.492 94.996) (width 0.4) (layer "B.Cu") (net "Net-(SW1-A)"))
 (segment (start 46.132 101.504) (end 89.82 101.504) (width 0.4) (layer "B.Cu") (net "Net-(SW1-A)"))
 (segment (start 41.148 96.52) (end 46.132 101.504) (width 0.4) (layer "B.Cu") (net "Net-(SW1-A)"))
 (segment (start 90.932 102.616) (end 99.06 102.616) (width 0.4) (layer "B.Cu") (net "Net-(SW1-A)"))
 (segment (start 89.82 101.504) (end 90.932 102.616) (width 0.4) (layer "B.Cu") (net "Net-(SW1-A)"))
 (segment (start 103.124 89.840444) (end 104.665186 88.299258) (width 0.4) (layer "B.Cu") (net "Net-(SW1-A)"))
 (segment (start 117.608242 88.299258) (end 119.888 90.579016) (width 0.4) (layer "B.Cu") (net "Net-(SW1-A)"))
 (segment (start 42.672 88.392) (end 41.148 89.916) (width 0.4) (layer "B.Cu") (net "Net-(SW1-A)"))
 (segment (start 41.148 89.916) (end 41.148 96.52) (width 0.4) (layer "B.Cu") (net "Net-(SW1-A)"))
 (segment (start 122.976 98.258292) (end 122.976 81.28) (width 0.4) (layer "B.Cu") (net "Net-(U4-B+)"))
 (segment (start 126.238708 101.521) (end 122.976 98.258292) (width 0.4) (layer "B.Cu") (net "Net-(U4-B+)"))
 (segment (start 124.46 91.742292) (end 124.46 86.868) (width 0.4) (layer "B.Cu") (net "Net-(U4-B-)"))
 (segment (start 126.238708 93.521) (end 124.46 91.742292) (width 0.4) (layer "B.Cu") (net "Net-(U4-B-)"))
 (segment (start 124.46 86.868) (end 125.476 85.852) (width 0.4) (layer "B.Cu") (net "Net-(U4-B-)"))
 (segment (start 125.476 85.852) (end 125.476 81.28) (width 0.4) (layer "B.Cu") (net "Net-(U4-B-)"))
 (segment (start 136.852 101.4) (end 136.852 97.536) (width 0.4) (layer "B.Cu") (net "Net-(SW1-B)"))
 (segment (start 133.731 104.521) (end 136.852 101.4) (width 0.4) (layer "B.Cu") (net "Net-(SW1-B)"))
 (segment (start 126.238708 104.521) (end 133.731 104.521) (width 0.4) (layer "B.Cu") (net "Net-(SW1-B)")))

